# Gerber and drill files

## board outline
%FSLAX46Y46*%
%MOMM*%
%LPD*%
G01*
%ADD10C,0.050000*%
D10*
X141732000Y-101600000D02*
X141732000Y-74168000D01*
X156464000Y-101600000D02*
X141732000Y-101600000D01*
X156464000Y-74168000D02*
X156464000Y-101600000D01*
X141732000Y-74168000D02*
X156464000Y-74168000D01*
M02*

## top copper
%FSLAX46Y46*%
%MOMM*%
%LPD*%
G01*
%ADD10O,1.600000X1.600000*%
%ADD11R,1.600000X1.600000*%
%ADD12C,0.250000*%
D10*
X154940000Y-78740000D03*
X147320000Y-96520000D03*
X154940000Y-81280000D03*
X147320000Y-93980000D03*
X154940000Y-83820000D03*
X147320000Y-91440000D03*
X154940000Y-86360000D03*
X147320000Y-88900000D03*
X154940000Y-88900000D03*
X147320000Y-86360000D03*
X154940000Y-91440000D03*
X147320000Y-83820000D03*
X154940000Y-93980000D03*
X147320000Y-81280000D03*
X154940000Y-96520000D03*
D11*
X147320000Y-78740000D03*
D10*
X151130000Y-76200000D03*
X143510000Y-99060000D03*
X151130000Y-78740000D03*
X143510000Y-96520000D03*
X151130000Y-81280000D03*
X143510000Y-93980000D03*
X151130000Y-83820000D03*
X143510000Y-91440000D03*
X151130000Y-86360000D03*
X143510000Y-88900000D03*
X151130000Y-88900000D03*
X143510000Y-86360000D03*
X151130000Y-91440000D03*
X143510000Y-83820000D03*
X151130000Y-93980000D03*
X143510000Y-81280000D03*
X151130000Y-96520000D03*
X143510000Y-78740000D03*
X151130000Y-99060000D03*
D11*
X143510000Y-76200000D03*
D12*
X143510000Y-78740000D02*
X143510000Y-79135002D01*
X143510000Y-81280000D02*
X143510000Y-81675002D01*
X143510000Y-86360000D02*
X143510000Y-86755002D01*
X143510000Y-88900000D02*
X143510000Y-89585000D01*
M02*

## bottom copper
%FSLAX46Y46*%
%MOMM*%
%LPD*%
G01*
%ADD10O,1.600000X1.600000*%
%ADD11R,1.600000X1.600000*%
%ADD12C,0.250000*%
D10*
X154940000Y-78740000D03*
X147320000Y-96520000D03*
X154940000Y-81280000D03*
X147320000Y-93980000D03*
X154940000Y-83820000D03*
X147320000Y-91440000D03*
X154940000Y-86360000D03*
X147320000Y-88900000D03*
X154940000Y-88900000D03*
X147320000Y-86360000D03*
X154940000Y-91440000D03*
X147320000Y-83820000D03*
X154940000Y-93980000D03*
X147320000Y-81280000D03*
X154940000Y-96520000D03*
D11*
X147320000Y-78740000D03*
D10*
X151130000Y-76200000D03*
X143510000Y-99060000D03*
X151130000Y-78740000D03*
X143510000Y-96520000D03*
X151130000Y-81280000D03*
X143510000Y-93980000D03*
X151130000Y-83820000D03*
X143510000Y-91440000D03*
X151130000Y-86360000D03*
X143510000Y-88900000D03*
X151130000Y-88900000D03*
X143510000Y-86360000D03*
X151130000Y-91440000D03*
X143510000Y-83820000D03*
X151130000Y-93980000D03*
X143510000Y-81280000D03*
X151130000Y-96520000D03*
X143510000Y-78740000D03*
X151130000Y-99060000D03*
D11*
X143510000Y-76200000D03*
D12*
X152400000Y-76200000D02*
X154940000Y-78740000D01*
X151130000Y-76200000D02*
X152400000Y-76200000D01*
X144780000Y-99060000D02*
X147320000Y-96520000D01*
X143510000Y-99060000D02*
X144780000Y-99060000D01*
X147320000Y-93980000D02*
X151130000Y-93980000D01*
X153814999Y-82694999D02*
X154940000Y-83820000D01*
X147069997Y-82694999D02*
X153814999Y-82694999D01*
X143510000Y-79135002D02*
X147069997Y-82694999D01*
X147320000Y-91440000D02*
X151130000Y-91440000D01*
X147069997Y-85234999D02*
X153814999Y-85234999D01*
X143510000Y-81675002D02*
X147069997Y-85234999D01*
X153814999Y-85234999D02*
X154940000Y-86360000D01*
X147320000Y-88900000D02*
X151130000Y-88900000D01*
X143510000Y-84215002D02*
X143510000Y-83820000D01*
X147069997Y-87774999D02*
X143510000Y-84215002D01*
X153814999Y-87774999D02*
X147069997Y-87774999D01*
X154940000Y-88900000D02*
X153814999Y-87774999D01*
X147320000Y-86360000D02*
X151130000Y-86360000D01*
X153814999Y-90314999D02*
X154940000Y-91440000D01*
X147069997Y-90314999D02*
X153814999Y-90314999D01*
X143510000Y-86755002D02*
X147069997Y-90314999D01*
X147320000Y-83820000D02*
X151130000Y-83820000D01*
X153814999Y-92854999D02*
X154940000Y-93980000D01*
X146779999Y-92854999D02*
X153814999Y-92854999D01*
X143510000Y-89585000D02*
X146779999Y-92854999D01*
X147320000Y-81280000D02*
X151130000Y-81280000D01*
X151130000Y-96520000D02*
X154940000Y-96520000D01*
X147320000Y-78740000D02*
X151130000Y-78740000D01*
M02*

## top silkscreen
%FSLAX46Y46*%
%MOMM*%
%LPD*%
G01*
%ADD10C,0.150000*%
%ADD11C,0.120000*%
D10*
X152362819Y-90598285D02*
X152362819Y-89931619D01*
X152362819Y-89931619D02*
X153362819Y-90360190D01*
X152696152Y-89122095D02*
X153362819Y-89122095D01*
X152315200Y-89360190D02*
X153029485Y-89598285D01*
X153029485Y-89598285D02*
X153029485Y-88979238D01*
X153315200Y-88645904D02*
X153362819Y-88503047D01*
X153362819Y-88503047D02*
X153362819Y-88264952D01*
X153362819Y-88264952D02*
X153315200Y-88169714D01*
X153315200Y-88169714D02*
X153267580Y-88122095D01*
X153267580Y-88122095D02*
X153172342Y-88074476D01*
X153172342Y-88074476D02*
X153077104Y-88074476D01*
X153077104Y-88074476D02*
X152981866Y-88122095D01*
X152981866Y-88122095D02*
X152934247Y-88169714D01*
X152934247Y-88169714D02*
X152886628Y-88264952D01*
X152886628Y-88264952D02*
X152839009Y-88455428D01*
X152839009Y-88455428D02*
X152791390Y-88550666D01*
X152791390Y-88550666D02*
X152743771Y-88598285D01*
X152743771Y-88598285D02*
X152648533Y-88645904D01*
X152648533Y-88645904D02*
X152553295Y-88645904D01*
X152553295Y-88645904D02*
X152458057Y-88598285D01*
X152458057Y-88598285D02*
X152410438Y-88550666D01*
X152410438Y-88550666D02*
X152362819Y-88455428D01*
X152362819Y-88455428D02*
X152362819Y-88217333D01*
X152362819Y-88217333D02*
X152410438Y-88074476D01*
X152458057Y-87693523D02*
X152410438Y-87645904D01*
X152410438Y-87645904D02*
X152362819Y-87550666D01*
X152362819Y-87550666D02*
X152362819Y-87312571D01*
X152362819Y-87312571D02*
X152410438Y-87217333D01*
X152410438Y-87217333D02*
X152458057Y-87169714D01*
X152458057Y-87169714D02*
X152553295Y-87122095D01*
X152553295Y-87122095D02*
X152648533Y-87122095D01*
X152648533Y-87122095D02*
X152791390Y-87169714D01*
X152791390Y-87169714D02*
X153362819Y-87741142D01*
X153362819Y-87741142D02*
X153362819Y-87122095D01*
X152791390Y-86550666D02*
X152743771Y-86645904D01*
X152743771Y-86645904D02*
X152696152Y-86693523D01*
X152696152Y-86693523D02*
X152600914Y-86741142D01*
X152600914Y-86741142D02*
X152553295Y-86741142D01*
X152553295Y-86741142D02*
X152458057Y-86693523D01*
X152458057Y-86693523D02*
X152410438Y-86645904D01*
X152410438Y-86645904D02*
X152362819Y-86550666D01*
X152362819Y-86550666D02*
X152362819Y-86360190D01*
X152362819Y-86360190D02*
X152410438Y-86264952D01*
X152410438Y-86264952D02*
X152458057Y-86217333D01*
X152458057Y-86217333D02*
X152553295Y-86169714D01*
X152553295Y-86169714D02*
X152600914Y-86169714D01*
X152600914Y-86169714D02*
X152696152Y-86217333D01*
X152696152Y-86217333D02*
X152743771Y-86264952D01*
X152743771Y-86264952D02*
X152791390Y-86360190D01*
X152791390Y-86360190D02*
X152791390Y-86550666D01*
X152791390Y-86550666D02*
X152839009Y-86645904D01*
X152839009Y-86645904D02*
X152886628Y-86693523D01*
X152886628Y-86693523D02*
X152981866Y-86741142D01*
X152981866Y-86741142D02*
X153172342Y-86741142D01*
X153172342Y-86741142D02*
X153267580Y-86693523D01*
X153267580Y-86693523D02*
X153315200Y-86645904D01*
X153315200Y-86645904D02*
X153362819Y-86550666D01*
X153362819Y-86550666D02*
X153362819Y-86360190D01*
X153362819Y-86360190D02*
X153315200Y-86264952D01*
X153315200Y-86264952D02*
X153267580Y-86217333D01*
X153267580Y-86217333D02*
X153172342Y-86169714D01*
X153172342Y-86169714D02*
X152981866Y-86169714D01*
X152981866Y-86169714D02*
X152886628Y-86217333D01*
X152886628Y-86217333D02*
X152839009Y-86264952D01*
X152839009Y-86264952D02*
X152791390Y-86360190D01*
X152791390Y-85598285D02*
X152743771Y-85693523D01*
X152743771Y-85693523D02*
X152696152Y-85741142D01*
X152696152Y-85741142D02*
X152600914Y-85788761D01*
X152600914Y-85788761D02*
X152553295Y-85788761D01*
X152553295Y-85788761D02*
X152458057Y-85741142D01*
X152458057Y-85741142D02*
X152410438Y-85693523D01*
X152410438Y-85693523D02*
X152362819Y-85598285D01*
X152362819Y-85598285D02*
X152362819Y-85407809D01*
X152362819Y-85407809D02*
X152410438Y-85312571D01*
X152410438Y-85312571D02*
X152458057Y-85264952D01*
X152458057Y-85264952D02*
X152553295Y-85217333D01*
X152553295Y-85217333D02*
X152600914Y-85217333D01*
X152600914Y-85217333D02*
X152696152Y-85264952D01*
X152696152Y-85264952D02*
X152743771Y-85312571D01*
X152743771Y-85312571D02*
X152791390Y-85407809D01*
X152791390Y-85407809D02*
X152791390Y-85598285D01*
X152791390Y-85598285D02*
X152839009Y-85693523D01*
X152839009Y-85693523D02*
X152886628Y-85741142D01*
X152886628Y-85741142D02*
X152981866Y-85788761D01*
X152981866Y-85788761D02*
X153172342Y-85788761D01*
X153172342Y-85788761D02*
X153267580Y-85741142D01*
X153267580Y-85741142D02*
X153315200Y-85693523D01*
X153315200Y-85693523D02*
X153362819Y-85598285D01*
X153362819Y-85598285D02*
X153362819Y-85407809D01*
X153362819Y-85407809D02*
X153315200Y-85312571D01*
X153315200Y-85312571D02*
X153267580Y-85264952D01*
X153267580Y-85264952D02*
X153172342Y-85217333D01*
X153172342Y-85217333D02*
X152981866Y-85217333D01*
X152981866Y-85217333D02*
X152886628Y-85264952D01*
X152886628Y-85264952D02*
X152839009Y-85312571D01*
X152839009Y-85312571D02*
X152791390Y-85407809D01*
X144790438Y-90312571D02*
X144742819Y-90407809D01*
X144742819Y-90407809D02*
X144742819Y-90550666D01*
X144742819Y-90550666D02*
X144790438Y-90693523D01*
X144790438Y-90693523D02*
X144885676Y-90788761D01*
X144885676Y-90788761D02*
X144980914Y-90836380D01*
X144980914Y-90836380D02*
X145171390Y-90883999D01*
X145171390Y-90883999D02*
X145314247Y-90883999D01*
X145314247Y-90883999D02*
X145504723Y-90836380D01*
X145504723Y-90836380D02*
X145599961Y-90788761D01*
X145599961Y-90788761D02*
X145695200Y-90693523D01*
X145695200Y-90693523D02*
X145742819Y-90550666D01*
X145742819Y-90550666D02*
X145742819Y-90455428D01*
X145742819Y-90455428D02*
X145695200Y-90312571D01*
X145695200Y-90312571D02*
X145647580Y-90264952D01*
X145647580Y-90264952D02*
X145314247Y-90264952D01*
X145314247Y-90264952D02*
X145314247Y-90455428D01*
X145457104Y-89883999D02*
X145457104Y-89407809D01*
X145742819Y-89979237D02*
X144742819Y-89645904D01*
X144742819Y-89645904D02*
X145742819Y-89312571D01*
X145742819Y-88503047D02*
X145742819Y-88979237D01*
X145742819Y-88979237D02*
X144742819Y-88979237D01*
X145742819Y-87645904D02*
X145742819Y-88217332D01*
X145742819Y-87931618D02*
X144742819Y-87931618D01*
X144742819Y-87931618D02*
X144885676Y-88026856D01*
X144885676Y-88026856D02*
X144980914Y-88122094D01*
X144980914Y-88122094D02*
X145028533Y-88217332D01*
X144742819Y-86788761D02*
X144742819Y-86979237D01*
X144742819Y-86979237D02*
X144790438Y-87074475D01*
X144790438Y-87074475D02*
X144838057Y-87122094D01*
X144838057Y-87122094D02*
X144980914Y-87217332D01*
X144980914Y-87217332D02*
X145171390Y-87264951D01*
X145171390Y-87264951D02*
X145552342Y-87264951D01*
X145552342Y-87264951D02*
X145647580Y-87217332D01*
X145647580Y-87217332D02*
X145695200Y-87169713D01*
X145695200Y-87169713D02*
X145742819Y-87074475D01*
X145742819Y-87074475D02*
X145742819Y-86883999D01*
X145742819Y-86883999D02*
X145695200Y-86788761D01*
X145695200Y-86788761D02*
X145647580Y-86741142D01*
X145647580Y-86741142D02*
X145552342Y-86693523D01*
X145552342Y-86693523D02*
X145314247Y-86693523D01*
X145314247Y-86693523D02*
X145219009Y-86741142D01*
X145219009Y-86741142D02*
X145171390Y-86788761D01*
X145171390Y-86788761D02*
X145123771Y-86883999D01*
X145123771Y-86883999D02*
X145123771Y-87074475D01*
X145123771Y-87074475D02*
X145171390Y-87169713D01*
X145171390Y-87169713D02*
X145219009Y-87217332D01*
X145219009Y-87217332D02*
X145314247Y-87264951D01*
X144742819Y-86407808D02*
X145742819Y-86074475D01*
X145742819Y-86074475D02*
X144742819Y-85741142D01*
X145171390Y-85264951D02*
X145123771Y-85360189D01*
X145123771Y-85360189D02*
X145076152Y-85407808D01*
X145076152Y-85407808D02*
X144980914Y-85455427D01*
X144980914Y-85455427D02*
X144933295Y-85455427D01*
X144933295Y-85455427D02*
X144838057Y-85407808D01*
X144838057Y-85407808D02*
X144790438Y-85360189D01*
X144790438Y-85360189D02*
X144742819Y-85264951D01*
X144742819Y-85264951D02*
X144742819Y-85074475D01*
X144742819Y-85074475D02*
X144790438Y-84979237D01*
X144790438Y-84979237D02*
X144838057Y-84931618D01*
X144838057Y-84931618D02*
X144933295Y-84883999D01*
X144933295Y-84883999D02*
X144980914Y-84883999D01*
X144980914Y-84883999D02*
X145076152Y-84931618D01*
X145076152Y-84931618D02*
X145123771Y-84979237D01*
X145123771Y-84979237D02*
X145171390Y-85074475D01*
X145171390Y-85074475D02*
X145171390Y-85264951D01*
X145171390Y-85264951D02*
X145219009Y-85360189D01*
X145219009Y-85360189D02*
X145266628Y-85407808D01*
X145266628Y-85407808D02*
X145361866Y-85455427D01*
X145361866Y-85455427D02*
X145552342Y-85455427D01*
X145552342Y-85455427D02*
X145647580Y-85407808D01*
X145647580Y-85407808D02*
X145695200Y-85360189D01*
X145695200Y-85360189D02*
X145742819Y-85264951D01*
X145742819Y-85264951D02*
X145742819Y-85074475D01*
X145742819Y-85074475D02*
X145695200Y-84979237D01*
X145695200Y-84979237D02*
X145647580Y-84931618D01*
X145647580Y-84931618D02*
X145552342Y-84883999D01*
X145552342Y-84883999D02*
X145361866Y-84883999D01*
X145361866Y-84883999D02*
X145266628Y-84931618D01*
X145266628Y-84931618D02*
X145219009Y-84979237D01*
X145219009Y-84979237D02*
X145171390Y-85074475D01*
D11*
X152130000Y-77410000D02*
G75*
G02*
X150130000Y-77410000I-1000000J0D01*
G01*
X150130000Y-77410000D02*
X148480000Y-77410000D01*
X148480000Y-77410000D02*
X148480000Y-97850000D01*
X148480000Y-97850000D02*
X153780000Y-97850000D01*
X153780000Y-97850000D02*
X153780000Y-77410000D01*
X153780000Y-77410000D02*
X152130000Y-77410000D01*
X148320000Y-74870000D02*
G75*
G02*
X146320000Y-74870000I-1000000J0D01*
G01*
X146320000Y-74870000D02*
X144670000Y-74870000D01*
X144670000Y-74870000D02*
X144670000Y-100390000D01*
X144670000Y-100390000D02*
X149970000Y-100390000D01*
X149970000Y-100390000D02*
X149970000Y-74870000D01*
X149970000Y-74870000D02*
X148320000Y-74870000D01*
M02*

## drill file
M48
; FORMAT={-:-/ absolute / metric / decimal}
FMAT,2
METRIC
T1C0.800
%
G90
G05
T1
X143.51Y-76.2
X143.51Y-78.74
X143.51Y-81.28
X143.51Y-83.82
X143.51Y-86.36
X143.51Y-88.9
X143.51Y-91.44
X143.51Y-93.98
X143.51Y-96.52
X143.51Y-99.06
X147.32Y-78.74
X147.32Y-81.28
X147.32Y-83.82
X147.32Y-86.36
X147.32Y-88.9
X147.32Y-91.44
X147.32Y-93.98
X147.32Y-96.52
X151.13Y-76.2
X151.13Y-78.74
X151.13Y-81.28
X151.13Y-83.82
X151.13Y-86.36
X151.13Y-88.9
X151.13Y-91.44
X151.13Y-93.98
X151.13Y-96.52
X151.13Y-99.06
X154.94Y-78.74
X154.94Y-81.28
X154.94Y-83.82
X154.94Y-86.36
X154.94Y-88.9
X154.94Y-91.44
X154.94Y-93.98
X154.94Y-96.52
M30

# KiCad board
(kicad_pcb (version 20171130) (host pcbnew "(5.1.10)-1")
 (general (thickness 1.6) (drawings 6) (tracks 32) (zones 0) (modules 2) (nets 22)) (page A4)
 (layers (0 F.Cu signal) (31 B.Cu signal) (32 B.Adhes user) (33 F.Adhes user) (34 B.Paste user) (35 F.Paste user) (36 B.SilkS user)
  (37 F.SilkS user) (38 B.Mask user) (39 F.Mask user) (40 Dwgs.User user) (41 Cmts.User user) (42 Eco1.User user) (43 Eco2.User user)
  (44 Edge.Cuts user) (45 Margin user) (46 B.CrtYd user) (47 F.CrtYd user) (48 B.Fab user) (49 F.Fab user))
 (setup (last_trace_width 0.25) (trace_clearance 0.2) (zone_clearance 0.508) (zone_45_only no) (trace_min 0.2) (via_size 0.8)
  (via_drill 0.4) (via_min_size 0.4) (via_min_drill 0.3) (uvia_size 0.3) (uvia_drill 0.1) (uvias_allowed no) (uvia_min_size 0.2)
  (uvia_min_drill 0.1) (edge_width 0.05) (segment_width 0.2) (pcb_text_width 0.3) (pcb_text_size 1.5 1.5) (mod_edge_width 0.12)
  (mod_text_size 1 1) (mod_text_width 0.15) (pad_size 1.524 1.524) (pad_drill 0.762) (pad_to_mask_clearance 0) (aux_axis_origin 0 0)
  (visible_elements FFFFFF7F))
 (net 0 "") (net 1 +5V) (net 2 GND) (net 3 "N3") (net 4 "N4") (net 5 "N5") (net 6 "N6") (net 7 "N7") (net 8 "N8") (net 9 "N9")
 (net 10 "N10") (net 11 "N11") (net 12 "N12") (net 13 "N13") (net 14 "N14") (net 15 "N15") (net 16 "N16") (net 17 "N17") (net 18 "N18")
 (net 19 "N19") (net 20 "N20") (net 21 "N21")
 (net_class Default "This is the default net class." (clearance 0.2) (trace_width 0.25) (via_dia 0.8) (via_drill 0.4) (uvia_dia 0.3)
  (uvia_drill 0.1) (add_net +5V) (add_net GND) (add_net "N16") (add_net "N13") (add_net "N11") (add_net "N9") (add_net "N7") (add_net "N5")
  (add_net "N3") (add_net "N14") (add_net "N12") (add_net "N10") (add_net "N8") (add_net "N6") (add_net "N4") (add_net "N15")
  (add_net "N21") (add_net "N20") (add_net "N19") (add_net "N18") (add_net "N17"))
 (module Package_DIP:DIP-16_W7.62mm (layer F.Cu) (at 147.32 78.74)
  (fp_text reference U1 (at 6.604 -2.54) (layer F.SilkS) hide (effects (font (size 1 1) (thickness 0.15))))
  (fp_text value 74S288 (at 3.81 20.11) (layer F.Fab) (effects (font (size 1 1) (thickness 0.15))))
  (fp_arc (start 3.81 -1.33) (end 2.81 -1.33) (angle -180) (layer F.SilkS) (width 0.12))
  (fp_line (start 2.81 -1.33) (end 1.16 -1.33) (layer F.SilkS) (width 0.12))
  (fp_line (start 1.16 -1.33) (end 1.16 19.11) (layer F.SilkS) (width 0.12))
  (fp_line (start 1.16 19.11) (end 6.46 19.11) (layer F.SilkS) (width 0.12))
  (fp_line (start 6.46 19.11) (end 6.46 -1.33) (layer F.SilkS) (width 0.12))
  (fp_line (start 6.46 -1.33) (end 4.81 -1.33) (layer F.SilkS) (width 0.12))
  (pad 16 thru_hole oval (at 7.62 0) (size 1.6 1.6) (drill 0.8) (layers *.Cu *.Mask) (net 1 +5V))
  (pad 8 thru_hole oval (at 0 17.78) (size 1.6 1.6) (drill 0.8) (layers *.Cu *.Mask) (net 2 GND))
  (pad 15 thru_hole oval (at 7.62 2.54) (size 1.6 1.6) (drill 0.8) (layers *.Cu *.Mask) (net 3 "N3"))
  (pad 7 thru_hole oval (at 0 15.24) (size 1.6 1.6) (drill 0.8) (layers *.Cu *.Mask) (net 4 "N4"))
  (pad 14 thru_hole oval (at 7.62 5.08) (size 1.6 1.6) (drill 0.8) (layers *.Cu *.Mask) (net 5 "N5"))
  (pad 6 thru_hole oval (at 0 12.7) (size 1.6 1.6) (drill 0.8) (layers *.Cu *.Mask) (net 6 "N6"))
  (pad 13 thru_hole oval (at 7.62 7.62) (size 1.6 1.6) (drill 0.8) (layers *.Cu *.Mask) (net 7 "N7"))
  (pad 5 thru_hole oval (at 0 10.16) (size 1.6 1.6) (drill 0.8) (layers *.Cu *.Mask) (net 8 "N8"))
  (pad 12 thru_hole oval (at 7.62 10.16) (size 1.6 1.6) (drill 0.8) (layers *.Cu *.Mask) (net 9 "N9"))
  (pad 4 thru_hole oval (at 0 7.62) (size 1.6 1.6) (drill 0.8) (layers *.Cu *.Mask) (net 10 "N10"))
  (pad 11 thru_hole oval (at 7.62 12.7) (size 1.6 1.6) (drill 0.8) (layers *.Cu *.Mask) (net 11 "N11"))
  (pad 3 thru_hole oval (at 0 5.08) (size 1.6 1.6) (drill 0.8) (layers *.Cu *.Mask) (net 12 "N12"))
  (pad 10 thru_hole oval (at 7.62 15.24) (size 1.6 1.6) (drill 0.8) (layers *.Cu *.Mask) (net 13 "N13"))
  (pad 2 thru_hole oval (at 0 2.54) (size 1.6 1.6) (drill 0.8) (layers *.Cu *.Mask) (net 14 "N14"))
  (pad 9 thru_hole oval (at 7.62 17.78) (size 1.6 1.6) (drill 0.8) (layers *.Cu *.Mask) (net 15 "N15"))
  (pad 1 thru_hole rect (at 0 0) (size 1.6 1.6) (drill 0.8) (layers *.Cu *.Mask) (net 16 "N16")))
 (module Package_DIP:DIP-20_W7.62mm (layer F.Cu) (at 143.51 76.2)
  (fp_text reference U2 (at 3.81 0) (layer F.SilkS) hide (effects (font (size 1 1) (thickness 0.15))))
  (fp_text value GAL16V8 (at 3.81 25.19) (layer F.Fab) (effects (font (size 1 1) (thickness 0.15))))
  (fp_arc (start 3.81 -1.33) (end 2.81 -1.33) (angle -180) (layer F.SilkS) (width 0.12))
  (fp_line (start 2.81 -1.33) (end 1.16 -1.33) (layer F.SilkS) (width 0.12))
  (fp_line (start 1.16 -1.33) (end 1.16 24.19) (layer F.SilkS) (width 0.12))
  (fp_line (start 1.16 24.19) (end 6.46 24.19) (layer F.SilkS) (width 0.12))
  (fp_line (start 6.46 24.19) (end 6.46 -1.33) (layer F.SilkS) (width 0.12))
  (fp_line (start 6.46 -1.33) (end 4.81 -1.33) (layer F.SilkS) (width 0.12))
  (pad 20 thru_hole oval (at 7.62 0) (size 1.6 1.6) (drill 0.8) (layers *.Cu *.Mask) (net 1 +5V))
  (pad 10 thru_hole oval (at 0 22.86) (size 1.6 1.6) (drill 0.8) (layers *.Cu *.Mask) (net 2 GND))
  (pad 19 thru_hole oval (at 7.62 2.54) (size 1.6 1.6) (drill 0.8) (layers *.Cu *.Mask) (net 16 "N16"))
  (pad 9 thru_hole oval (at 0 20.32) (size 1.6 1.6) (drill 0.8) (layers *.Cu *.Mask) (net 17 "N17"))
  (pad 18 thru_hole oval (at 7.62 5.08) (size 1.6 1.6) (drill 0.8) (layers *.Cu *.Mask) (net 14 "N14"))
  (pad 8 thru_hole oval (at 0 17.78) (size 1.6 1.6) (drill 0.8) (layers *.Cu *.Mask) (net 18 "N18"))
  (pad 17 thru_hole oval (at 7.62 7.62) (size 1.6 1.6) (drill 0.8) (layers *.Cu *.Mask) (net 12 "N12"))
  (pad 7 thru_hole oval (at 0 15.24) (size 1.6 1.6) (drill 0.8) (layers *.Cu *.Mask) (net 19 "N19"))
  (pad 16 thru_hole oval (at 7.62 10.16) (size 1.6 1.6) (drill 0.8) (layers *.Cu *.Mask) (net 10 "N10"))
  (pad 6 thru_hole oval (at 0 12.7) (size 1.6 1.6) (drill 0.8) (layers *.Cu *.Mask) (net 13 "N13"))
  (pad 15 thru_hole oval (at 7.62 12.7) (size 1.6 1.6) (drill 0.8) (layers *.Cu *.Mask) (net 8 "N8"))
  (pad 5 thru_hole oval (at 0 10.16) (size 1.6 1.6) (drill 0.8) (layers *.Cu *.Mask) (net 11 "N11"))
  (pad 14 thru_hole oval (at 7.62 15.24) (size 1.6 1.6) (drill 0.8) (layers *.Cu *.Mask) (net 6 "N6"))
  (pad 4 thru_hole oval (at 0 7.62) (size 1.6 1.6) (drill 0.8) (layers *.Cu *.Mask) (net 9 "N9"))
  (pad 13 thru_hole oval (at 7.62 17.78) (size 1.6 1.6) (drill 0.8) (layers *.Cu *.Mask) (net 4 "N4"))
  (pad 3 thru_hole oval (at 0 5.08) (size 1.6 1.6) (drill 0.8) (layers *.Cu *.Mask) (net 7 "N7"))
  (pad 12 thru_hole oval (at 7.62 20.32) (size 1.6 1.6) (drill 0.8) (layers *.Cu *.Mask) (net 15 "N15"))
  (pad 2 thru_hole oval (at 0 2.54) (size 1.6 1.6) (drill 0.8) (layers *.Cu *.Mask) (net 5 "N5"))
  (pad 11 thru_hole oval (at 7.62 22.86) (size 1.6 1.6) (drill 0.8) (layers *.Cu *.Mask) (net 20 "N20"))
  (pad 1 thru_hole rect (at 0 0) (size 1.6 1.6) (drill 0.8) (layers *.Cu *.Mask) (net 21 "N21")))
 (gr_line (start 141.732 101.6) (end 141.732 74.168) (layer Edge.Cuts) (width 0.05))
 (gr_line (start 156.464 101.6) (end 141.732 101.6) (layer Edge.Cuts) (width 0.05))
 (gr_line (start 156.464 74.168) (end 156.464 101.6) (layer Edge.Cuts) (width 0.05))
 (gr_line (start 141.732 74.168) (end 156.464 74.168) (layer Edge.Cuts) (width 0.05))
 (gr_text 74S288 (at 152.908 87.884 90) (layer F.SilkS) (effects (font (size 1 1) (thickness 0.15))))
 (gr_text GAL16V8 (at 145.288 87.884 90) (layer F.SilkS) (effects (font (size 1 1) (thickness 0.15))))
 (segment (start 152.4 76.2) (end 154.94 78.74) (width 0.25) (layer B.Cu) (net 1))
 (segment (start 151.13 76.2) (end 152.4 76.2) (width 0.25) (layer B.Cu) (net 1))
 (segment (start 144.78 99.06) (end 147.32 96.52) (width 0.25) (layer B.Cu) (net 2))
 (segment (start 143.51 99.06) (end 144.78 99.06) (width 0.25) (layer B.Cu) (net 2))
 (segment (start 147.32 93.98) (end 151.13 93.98) (width 0.25) (layer B.Cu) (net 4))
 (segment (start 153.814999 82.694999) (end 154.94 83.82) (width 0.25) (layer B.Cu) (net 5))
 (segment (start 147.069997 82.694999) (end 153.814999 82.694999) (width 0.25) (layer B.Cu) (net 5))
 (segment (start 143.51 79.135002) (end 147.069997 82.694999) (width 0.25) (layer B.Cu) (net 5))
 (segment (start 143.51 78.74) (end 143.51 79.135002) (width 0.25) (layer F.Cu) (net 5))
 (segment (start 147.32 91.44) (end 151.13 91.44) (width 0.25) (layer B.Cu) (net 6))
 (segment (start 147.069997 85.234999) (end 153.814999 85.234999) (width 0.25) (layer B.Cu) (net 7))
 (segment (start 143.51 81.675002) (end 147.069997 85.234999) (width 0.25) (layer B.Cu) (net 7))
 (segment (start 143.51 81.28) (end 143.51 81.675002) (width 0.25) (layer F.Cu) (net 7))
 (segment (start 153.814999 85.234999) (end 154.94 86.36) (width 0.25) (layer B.Cu) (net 7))
 (segment (start 147.32 88.9) (end 151.13 88.9) (width 0.25) (layer B.Cu) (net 8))
 (segment (start 143.51 84.215002) (end 143.51 83.82) (width 0.25) (layer B.Cu) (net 9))
 (segment (start 147.069997 87.774999) (end 143.51 84.215002) (width 0.25) (layer B.Cu) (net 9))
 (segment (start 153.814999 87.774999) (end 147.069997 87.774999) (width 0.25) (layer B.Cu) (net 9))
 (segment (start 154.94 88.9) (end 153.814999 87.774999) (width 0.25) (layer B.Cu) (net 9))
 (segment (start 147.32 86.36) (end 151.13 86.36) (width 0.25) (layer B.Cu) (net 10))
 (segment (start 153.814999 90.314999) (end 154.94 91.44) (width 0.25) (layer B.Cu) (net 11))
 (segment (start 147.069997 90.314999) (end 153.814999 90.314999) (width 0.25) (layer B.Cu) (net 11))
 (segment (start 143.51 86.755002) (end 147.069997 90.314999) (width 0.25) (layer B.Cu) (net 11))
 (segment (start 143.51 86.36) (end 143.51 86.755002) (width 0.25) (layer F.Cu) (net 11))
 (segment (start 147.32 83.82) (end 151.13 83.82) (width 0.25) (layer B.Cu) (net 12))
 (segment (start 153.814999 92.854999) (end 154.94 93.98) (width 0.25) (layer B.Cu) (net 13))
 (segment (start 146.779999 92.854999) (end 153.814999 92.854999) (width 0.25) (layer B.Cu) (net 13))
 (segment (start 143.51 89.585) (end 146.779999 92.854999) (width 0.25) (layer B.Cu) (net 13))
 (segment (start 143.51 88.9) (end 143.51 89.585) (width 0.25) (layer F.Cu) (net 13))
 (segment (start 147.32 81.28) (end 151.13 81.28) (width 0.25) (layer B.Cu) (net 14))
 (segment (start 151.13 96.52) (end 154.94 96.52) (width 0.25) (layer B.Cu) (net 15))
 (segment (start 147.32 78.74) (end 151.13 78.74) (width 0.25) (layer B.Cu) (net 16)))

